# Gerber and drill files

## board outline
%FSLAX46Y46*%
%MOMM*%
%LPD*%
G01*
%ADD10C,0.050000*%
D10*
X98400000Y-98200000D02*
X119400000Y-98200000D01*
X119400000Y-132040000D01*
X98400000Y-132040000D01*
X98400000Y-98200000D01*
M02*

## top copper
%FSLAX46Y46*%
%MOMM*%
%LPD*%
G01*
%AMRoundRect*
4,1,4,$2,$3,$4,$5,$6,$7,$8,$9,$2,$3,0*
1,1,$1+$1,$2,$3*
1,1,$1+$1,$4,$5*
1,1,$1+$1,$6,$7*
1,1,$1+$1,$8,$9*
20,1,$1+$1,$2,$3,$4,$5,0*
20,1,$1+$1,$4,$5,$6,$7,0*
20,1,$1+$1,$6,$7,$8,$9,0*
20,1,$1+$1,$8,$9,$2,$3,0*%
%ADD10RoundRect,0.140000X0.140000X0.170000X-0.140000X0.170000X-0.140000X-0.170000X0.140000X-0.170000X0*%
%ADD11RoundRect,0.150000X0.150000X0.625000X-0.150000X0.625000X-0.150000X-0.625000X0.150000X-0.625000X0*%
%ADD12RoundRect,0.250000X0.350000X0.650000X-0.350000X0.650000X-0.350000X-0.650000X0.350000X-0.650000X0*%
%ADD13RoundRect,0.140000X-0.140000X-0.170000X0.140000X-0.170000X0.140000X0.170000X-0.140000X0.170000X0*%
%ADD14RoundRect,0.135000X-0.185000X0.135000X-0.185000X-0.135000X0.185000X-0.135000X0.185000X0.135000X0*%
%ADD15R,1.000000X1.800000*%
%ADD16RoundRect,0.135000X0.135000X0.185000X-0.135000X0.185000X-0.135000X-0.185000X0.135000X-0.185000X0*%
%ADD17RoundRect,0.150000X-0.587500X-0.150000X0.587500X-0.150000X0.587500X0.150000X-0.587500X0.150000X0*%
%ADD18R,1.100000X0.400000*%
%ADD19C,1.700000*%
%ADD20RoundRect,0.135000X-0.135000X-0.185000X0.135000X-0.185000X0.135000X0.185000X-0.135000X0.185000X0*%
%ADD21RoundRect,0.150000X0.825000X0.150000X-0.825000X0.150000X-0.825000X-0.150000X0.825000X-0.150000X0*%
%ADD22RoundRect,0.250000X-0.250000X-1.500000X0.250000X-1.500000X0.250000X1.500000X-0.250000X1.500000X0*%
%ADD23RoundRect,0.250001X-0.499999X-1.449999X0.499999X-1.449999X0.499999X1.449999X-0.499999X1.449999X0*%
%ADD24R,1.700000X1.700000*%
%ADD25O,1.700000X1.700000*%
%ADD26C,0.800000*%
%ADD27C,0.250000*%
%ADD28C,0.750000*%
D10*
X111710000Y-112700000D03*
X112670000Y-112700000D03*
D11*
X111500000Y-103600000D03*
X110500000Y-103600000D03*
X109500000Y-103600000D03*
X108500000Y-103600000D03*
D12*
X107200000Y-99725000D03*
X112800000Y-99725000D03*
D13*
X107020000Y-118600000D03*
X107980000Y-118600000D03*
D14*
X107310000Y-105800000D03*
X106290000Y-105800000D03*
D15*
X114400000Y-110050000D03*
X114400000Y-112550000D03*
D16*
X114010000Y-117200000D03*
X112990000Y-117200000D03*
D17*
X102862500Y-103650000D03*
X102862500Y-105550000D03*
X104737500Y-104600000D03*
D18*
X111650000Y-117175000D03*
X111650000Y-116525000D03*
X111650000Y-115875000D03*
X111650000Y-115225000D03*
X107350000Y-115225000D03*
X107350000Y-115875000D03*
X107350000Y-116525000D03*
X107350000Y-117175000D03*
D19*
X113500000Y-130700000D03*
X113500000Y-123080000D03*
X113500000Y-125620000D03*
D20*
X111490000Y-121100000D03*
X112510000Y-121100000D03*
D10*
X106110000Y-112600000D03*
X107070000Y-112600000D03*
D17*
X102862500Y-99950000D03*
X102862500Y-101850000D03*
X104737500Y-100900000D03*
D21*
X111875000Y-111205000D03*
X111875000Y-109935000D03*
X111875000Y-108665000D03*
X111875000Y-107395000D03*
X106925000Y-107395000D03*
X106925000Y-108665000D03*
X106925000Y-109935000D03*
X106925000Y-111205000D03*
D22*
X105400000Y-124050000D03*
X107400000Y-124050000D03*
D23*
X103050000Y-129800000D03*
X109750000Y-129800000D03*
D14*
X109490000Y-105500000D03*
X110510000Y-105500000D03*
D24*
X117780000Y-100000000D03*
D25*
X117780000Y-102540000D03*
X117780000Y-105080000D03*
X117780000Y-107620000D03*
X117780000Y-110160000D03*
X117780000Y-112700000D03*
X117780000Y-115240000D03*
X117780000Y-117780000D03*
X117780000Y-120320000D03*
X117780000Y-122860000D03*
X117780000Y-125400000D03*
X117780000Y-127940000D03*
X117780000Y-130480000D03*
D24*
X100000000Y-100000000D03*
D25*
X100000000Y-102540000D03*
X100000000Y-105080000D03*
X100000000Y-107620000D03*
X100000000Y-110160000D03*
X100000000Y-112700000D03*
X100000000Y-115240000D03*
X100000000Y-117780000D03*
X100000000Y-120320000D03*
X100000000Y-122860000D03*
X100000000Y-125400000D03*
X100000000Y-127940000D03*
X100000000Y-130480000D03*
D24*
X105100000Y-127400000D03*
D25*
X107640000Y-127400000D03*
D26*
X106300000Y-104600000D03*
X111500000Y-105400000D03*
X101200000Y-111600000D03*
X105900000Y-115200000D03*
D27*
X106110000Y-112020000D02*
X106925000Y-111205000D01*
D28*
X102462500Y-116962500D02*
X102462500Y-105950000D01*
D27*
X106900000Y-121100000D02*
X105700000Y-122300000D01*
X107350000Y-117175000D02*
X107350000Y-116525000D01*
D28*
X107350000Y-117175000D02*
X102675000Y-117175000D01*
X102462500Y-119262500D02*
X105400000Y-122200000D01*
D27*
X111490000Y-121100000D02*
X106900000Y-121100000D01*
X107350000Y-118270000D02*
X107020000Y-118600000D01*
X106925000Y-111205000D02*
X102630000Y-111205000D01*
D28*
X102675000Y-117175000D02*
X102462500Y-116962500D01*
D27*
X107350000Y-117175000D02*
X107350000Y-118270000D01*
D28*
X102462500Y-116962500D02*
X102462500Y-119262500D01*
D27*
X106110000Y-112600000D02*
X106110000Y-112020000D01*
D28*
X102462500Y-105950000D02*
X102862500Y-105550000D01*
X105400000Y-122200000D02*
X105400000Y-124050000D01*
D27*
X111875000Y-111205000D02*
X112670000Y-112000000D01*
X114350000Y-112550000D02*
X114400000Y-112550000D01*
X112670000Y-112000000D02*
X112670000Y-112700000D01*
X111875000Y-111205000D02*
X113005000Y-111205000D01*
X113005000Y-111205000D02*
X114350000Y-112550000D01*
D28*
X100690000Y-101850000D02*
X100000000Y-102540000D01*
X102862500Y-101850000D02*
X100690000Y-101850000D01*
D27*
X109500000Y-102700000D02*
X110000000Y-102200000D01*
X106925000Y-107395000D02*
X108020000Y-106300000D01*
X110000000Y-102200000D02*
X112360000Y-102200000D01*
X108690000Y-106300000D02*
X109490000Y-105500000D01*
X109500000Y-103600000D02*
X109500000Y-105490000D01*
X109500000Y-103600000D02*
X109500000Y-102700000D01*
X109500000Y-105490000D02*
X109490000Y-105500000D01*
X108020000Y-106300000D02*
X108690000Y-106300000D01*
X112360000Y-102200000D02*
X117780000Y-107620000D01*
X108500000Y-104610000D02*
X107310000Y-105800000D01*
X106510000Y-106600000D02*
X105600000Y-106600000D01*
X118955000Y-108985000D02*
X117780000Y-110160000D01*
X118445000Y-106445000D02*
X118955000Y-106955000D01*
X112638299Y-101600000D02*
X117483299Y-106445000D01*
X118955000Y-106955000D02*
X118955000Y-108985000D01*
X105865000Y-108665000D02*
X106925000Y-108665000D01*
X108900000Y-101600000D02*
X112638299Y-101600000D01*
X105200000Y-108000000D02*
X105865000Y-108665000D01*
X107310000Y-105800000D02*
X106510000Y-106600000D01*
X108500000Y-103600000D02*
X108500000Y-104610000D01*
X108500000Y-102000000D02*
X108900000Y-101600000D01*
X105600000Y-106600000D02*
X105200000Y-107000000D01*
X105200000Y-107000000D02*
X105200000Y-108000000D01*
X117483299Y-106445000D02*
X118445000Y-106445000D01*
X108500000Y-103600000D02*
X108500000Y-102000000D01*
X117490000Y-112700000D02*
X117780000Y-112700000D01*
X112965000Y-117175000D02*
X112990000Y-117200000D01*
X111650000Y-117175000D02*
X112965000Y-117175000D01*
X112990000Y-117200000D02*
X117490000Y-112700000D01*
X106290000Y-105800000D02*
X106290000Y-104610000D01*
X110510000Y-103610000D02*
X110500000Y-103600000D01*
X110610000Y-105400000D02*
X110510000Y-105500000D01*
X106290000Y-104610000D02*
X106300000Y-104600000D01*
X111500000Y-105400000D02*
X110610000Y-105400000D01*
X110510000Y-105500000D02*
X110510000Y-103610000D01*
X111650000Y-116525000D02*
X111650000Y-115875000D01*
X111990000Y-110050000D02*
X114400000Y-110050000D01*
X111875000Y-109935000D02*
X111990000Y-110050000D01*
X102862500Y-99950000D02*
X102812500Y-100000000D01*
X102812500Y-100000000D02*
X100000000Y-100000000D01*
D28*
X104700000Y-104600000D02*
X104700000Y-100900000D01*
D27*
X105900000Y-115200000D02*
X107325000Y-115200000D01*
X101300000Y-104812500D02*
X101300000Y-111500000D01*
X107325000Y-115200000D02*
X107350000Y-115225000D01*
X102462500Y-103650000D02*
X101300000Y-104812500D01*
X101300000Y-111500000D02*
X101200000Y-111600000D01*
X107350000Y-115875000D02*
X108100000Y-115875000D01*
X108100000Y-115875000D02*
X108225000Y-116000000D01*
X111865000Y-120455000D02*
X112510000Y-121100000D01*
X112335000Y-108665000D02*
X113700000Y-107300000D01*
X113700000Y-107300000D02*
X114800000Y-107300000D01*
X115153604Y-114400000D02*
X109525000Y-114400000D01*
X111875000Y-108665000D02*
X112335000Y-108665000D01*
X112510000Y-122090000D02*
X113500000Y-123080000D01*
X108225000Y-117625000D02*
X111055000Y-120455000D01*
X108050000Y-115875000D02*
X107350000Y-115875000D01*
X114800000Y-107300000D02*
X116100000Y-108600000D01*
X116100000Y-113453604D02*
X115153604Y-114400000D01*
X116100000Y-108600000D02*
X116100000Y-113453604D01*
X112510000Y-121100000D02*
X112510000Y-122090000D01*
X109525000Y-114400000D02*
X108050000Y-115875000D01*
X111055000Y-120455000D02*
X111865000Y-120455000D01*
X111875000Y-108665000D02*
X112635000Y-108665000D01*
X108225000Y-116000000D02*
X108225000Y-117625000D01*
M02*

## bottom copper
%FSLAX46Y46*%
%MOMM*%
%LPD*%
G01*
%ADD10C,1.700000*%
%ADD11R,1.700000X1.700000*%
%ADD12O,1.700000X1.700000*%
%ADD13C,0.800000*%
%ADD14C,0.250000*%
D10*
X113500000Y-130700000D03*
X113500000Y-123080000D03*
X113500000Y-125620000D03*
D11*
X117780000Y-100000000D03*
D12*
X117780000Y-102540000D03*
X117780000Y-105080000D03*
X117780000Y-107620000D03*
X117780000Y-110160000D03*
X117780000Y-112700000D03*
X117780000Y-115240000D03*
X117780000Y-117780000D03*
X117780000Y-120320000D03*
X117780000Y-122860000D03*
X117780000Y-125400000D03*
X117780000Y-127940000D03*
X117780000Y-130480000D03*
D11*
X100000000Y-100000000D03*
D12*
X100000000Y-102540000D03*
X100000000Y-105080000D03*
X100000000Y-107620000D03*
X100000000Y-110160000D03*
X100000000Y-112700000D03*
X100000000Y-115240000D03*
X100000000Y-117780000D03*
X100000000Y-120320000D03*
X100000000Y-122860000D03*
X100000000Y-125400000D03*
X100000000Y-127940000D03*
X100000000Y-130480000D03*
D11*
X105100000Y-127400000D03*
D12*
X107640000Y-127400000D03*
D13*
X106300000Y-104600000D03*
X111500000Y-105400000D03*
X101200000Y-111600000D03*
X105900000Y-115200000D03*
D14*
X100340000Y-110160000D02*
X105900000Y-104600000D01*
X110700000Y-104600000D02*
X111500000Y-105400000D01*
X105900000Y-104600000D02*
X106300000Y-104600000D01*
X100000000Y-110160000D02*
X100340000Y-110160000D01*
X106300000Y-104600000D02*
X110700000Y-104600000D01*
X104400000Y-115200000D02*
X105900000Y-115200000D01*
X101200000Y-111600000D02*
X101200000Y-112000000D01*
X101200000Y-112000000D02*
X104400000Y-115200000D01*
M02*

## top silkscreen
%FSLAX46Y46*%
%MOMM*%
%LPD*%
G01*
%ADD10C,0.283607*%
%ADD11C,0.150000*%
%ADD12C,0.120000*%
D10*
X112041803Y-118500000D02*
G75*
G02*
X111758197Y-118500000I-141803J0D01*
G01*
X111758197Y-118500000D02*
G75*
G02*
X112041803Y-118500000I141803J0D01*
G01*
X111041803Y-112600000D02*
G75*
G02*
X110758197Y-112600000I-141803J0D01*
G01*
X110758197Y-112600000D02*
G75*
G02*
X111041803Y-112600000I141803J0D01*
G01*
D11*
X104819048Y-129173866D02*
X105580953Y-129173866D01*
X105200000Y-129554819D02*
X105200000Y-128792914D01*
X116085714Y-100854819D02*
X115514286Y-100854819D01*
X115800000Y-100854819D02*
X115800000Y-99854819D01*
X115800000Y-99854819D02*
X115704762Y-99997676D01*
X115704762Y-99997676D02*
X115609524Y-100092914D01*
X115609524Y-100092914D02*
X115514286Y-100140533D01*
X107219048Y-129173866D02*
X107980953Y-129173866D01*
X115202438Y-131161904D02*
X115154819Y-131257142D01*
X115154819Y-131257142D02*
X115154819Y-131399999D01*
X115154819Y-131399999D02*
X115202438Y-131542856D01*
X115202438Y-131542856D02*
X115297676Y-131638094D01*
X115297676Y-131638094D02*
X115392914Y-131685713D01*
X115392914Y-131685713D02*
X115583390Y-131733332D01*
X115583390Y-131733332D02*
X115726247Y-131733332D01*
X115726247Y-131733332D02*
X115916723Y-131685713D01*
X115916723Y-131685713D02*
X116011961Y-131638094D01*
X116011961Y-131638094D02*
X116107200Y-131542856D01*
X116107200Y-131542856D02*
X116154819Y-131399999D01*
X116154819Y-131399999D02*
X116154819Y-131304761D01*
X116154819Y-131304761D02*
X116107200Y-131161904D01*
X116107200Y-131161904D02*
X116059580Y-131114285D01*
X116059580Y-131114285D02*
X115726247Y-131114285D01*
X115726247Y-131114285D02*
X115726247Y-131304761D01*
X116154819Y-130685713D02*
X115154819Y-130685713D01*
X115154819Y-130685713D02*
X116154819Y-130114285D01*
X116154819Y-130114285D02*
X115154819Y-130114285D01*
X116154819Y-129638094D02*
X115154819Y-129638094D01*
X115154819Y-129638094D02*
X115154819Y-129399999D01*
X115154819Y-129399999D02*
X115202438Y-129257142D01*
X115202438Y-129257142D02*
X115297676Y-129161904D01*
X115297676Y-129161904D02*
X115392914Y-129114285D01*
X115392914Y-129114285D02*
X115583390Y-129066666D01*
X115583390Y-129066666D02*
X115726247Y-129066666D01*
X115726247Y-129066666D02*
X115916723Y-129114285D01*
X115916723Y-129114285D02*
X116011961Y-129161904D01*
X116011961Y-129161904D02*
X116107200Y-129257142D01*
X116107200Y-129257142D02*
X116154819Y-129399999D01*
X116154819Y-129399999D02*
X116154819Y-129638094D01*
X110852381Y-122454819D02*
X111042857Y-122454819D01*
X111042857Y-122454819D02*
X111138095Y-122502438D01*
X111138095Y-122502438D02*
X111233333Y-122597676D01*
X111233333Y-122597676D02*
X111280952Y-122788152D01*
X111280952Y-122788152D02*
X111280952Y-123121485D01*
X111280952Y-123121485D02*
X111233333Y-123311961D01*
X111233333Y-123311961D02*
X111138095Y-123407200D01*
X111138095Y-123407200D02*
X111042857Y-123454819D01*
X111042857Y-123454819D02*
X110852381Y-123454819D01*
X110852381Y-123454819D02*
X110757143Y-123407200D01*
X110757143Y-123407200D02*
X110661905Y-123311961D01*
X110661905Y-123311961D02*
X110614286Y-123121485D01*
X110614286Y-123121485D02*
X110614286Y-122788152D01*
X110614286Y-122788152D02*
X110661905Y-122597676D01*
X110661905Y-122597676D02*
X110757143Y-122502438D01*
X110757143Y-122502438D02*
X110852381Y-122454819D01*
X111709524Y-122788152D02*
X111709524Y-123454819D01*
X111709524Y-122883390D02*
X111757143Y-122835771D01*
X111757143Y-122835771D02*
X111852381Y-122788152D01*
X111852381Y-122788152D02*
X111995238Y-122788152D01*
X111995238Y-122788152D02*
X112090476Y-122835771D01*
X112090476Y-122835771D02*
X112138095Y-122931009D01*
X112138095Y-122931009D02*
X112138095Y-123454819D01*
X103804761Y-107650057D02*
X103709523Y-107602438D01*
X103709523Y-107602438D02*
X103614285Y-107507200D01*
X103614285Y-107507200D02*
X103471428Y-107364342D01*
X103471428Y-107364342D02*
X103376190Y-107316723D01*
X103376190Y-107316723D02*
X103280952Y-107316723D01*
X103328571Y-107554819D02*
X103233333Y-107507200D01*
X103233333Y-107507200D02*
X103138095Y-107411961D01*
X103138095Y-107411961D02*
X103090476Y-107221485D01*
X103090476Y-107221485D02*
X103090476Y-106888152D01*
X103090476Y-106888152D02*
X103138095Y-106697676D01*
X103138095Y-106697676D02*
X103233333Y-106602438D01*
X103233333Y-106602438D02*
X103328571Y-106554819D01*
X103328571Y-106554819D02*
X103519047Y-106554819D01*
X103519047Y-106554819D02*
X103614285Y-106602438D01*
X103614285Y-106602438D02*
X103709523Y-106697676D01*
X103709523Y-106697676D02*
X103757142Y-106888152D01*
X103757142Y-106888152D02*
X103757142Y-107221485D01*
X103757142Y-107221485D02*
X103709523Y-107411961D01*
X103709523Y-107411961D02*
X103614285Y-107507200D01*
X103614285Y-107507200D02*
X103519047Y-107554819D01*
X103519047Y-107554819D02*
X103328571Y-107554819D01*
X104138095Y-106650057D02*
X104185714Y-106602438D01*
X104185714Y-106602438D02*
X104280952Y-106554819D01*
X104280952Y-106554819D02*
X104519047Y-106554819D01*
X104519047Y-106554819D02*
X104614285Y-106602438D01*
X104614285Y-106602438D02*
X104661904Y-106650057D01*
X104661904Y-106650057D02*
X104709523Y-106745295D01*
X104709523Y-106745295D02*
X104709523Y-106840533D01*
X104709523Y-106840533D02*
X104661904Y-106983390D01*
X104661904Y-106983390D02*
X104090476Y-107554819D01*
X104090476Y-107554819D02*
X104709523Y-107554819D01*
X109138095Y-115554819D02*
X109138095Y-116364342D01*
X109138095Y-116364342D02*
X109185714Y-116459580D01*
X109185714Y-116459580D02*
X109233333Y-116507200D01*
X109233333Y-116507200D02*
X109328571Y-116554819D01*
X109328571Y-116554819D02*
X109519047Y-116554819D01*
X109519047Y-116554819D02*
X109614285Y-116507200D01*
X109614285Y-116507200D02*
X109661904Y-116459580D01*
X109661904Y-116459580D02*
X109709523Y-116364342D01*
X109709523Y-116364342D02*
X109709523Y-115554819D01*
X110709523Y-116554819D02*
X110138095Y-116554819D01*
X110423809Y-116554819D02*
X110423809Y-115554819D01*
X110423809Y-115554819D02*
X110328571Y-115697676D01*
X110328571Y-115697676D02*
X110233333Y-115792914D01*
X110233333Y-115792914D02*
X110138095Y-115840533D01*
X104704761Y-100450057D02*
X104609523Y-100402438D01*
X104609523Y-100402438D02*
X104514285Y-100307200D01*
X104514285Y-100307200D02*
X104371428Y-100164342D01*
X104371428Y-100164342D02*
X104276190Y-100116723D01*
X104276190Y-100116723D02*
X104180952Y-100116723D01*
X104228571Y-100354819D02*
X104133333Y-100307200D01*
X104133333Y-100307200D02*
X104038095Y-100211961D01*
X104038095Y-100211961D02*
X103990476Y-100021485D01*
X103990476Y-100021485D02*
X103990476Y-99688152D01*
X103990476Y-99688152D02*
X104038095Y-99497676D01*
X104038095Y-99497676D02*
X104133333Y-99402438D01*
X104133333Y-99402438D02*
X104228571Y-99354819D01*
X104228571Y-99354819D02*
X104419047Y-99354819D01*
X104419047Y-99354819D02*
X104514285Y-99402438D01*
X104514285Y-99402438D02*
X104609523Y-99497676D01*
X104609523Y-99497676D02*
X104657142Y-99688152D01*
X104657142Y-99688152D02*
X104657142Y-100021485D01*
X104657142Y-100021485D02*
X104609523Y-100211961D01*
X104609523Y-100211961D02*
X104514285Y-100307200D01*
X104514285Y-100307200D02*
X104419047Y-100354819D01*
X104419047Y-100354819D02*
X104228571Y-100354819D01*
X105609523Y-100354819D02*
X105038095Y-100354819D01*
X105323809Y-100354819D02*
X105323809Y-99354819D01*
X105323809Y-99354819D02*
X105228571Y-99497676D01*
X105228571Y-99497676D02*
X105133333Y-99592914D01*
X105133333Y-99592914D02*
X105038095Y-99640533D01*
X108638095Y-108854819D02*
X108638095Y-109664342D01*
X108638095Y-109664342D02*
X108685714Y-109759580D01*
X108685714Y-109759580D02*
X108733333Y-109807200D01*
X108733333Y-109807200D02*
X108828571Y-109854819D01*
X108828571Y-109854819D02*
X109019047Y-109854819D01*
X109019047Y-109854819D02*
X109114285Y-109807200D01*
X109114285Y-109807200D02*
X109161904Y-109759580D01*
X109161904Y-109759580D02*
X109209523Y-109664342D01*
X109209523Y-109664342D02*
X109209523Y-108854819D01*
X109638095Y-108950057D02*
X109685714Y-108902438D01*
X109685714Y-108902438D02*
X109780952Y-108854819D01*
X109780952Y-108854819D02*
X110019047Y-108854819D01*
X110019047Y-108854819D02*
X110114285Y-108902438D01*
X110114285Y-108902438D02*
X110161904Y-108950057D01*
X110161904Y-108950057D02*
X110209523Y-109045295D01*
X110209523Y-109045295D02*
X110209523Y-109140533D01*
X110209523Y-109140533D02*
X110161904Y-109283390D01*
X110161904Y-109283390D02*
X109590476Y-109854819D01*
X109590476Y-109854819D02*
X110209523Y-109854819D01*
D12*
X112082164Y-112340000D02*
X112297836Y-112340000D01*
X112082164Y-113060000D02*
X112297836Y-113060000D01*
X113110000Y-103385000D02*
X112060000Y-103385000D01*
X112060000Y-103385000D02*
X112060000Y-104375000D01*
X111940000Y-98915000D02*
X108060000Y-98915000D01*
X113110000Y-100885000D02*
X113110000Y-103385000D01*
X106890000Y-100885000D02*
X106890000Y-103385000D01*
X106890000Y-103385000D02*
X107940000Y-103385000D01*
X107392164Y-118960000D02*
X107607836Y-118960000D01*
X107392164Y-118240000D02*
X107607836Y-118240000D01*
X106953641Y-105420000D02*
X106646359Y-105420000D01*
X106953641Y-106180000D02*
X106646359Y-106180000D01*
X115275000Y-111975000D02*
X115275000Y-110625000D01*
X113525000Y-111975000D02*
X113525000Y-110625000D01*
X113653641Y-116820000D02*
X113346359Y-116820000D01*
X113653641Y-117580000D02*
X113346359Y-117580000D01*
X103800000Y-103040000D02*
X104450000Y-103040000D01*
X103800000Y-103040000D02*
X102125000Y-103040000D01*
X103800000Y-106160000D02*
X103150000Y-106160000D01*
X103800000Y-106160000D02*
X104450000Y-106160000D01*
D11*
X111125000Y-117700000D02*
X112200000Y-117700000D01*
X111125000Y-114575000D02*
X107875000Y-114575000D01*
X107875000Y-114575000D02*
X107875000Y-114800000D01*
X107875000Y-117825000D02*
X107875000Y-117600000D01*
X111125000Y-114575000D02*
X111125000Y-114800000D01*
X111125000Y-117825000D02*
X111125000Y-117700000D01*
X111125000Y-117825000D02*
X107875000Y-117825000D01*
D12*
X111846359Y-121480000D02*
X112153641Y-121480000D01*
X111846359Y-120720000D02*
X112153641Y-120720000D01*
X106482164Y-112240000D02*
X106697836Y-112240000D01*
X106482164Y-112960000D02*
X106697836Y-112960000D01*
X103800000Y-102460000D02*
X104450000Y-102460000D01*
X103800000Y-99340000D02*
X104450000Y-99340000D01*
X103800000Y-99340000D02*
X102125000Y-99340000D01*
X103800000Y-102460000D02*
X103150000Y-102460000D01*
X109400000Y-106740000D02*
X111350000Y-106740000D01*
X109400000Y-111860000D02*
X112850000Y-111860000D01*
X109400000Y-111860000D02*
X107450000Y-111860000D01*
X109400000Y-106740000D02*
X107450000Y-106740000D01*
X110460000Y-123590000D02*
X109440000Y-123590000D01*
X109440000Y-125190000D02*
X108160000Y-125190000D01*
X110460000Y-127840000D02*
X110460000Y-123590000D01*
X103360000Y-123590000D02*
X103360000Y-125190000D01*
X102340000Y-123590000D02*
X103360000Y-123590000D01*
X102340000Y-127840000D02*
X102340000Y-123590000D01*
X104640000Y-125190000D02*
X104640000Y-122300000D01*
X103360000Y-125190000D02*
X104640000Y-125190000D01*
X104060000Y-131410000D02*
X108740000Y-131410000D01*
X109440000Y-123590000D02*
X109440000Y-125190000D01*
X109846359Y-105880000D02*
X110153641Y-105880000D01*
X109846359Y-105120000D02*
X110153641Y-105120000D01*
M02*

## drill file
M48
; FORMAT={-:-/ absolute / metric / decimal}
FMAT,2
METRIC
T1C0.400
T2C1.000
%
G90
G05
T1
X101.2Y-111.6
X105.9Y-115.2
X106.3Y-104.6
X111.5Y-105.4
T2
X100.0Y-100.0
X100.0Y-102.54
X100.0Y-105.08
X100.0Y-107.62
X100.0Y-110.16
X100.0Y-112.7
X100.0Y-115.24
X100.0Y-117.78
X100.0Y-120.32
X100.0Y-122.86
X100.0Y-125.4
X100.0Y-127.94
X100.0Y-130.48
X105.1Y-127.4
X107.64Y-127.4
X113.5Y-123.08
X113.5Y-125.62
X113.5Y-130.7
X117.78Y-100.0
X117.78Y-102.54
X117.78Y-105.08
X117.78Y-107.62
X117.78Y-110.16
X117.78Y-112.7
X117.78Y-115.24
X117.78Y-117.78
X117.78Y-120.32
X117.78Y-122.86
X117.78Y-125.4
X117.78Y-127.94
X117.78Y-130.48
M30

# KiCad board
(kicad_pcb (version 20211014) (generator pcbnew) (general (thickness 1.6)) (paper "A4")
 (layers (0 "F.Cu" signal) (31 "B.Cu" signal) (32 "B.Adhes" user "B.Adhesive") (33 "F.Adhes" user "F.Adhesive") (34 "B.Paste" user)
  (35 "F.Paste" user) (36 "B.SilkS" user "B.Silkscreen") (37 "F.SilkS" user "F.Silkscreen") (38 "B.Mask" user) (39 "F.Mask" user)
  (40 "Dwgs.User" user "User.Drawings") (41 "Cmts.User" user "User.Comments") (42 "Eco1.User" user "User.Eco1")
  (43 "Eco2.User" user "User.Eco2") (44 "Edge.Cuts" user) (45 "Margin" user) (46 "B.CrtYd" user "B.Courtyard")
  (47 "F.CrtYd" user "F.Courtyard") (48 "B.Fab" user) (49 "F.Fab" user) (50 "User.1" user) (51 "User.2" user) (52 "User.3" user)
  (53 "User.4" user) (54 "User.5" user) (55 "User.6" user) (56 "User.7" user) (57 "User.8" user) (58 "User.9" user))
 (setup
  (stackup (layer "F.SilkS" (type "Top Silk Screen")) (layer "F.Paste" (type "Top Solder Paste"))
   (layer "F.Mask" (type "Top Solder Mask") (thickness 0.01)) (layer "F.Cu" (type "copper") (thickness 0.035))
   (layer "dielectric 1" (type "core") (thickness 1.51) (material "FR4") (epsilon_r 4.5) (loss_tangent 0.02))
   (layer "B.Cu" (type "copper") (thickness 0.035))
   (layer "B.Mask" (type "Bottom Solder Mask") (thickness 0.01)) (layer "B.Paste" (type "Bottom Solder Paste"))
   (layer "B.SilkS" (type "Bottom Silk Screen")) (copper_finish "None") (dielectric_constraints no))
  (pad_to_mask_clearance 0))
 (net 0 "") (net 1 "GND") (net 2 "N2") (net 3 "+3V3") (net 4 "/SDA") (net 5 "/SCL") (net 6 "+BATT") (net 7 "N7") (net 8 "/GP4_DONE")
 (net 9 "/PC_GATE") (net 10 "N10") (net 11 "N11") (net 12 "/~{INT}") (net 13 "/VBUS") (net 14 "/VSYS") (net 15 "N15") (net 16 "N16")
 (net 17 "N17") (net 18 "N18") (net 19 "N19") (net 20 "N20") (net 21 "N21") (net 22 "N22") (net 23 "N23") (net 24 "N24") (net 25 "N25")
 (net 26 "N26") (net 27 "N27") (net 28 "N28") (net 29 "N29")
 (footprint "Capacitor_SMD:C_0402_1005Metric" (layer "F.Cu") (at 112.19 112.7)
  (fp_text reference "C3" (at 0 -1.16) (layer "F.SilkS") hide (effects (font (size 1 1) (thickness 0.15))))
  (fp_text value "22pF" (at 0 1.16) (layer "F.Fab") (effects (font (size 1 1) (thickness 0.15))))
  (fp_line (start -0.107836 -0.36) (end 0.107836 -0.36) (layer "F.SilkS") (width 0.12))
  (fp_line (start -0.107836 0.36) (end 0.107836 0.36) (layer "F.SilkS") (width 0.12))
  (pad "1" smd roundrect (at -0.48 0 180) (size 0.56 0.62) (layers "F.Cu" "F.Paste" "F.Mask") (roundrect_rratio 0.25) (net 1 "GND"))
  (pad "2" smd roundrect (at 0.48 0 180) (size 0.56 0.62) (layers "F.Cu" "F.Paste" "F.Mask") (roundrect_rratio 0.25) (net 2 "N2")))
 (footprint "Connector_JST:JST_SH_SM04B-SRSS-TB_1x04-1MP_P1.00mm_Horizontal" (layer "F.Cu") (at 110 101.6 180)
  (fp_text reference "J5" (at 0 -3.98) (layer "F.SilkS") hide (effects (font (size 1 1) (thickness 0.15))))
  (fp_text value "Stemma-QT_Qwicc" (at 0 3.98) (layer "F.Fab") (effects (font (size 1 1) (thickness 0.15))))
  (fp_line (start -3.11 -1.785) (end -2.06 -1.785) (layer "F.SilkS") (width 0.12))
  (fp_line (start -2.06 -1.785) (end -2.06 -2.775) (layer "F.SilkS") (width 0.12))
  (fp_line (start -1.94 2.685) (end 1.94 2.685) (layer "F.SilkS") (width 0.12))
  (fp_line (start -3.11 0.715) (end -3.11 -1.785) (layer "F.SilkS") (width 0.12))
  (fp_line (start 3.11 0.715) (end 3.11 -1.785) (layer "F.SilkS") (width 0.12))
  (fp_line (start 3.11 -1.785) (end 2.06 -1.785) (layer "F.SilkS") (width 0.12))
  (pad "1" smd roundrect (at -1.5 -2 180) (size 0.6 1.55) (layers "F.Cu" "F.Paste" "F.Mask") (roundrect_rratio 0.25) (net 1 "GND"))
  (pad "2" smd roundrect (at -0.5 -2 180) (size 0.6 1.55) (layers "F.Cu" "F.Paste" "F.Mask") (roundrect_rratio 0.25) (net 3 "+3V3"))
  (pad "3" smd roundrect (at 0.5 -2 180) (size 0.6 1.55) (layers "F.Cu" "F.Paste" "F.Mask") (roundrect_rratio 0.25) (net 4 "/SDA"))
  (pad "4" smd roundrect (at 1.5 -2 180) (size 0.6 1.55) (layers "F.Cu" "F.Paste" "F.Mask") (roundrect_rratio 0.25) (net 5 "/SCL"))
  (pad "MP" smd roundrect (at 2.8 1.875 180) (size 1.2 1.8) (layers "F.Cu" "F.Paste" "F.Mask") (roundrect_rratio 0.208333))
  (pad "MP" smd roundrect (at -2.8 1.875 180) (size 1.2 1.8) (layers "F.Cu" "F.Paste" "F.Mask") (roundrect_rratio 0.208333)))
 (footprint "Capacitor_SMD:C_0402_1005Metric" (layer "F.Cu") (at 107.5 118.6)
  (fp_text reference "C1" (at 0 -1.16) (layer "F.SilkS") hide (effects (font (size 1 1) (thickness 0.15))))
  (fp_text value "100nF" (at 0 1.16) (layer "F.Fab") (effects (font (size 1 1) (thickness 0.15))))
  (fp_line (start -0.107836 0.36) (end 0.107836 0.36) (layer "F.SilkS") (width 0.12))
  (fp_line (start -0.107836 -0.36) (end 0.107836 -0.36) (layer "F.SilkS") (width 0.12))
  (pad "1" smd roundrect (at -0.48 0) (size 0.56 0.62) (layers "F.Cu" "F.Paste" "F.Mask") (roundrect_rratio 0.25) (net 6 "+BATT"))
  (pad "2" smd roundrect (at 0.48 0) (size 0.56 0.62) (layers "F.Cu" "F.Paste" "F.Mask") (roundrect_rratio 0.25) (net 1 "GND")))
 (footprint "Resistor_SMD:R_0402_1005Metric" (layer "F.Cu") (at 106.8 105.8 180)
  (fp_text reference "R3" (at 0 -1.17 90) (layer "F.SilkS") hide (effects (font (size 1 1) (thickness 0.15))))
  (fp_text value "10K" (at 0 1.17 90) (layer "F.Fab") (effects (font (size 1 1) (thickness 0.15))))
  (fp_line (start -0.153641 0.38) (end 0.153641 0.38) (layer "F.SilkS") (width 0.12))
  (fp_line (start -0.153641 -0.38) (end 0.153641 -0.38) (layer "F.SilkS") (width 0.12))
  (pad "1" smd roundrect (at -0.51 0 270) (size 0.54 0.64) (layers "F.Cu" "F.Paste" "F.Mask") (roundrect_rratio 0.25) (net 5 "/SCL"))
  (pad "2" smd roundrect (at 0.51 0 270) (size 0.54 0.64) (layers "F.Cu" "F.Paste" "F.Mask") (roundrect_rratio 0.25) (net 3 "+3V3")))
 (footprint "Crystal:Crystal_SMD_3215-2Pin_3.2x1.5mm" (layer "F.Cu") (at 114.4 111.3 90)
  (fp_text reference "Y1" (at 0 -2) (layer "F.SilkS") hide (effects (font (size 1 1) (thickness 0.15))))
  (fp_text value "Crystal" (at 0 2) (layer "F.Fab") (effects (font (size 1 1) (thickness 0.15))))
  (fp_line (start -0.675 0.875) (end 0.675 0.875) (layer "F.SilkS") (width 0.12))
  (fp_line (start -0.675 -0.875) (end 0.675 -0.875) (layer "F.SilkS") (width 0.12))
  (pad "1" smd rect (at 1.25 0 180) (size 1 1.8) (layers "F.Cu" "F.Paste" "F.Mask") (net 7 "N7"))
  (pad "2" smd rect (at -1.25 0 180) (size 1 1.8) (layers "F.Cu" "F.Paste" "F.Mask") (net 2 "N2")))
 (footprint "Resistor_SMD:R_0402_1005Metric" (layer "F.Cu") (at 113.5 117.2 180)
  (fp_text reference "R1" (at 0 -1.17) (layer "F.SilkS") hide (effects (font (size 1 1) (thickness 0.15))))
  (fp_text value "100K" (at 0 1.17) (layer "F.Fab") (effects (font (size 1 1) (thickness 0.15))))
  (fp_line (start -0.153641 0.38) (end 0.153641 0.38) (layer "F.SilkS") (width 0.12))
  (fp_line (start -0.153641 -0.38) (end 0.153641 -0.38) (layer "F.SilkS") (width 0.12))
  (pad "1" smd roundrect (at -0.51 0 180) (size 0.54 0.64) (layers "F.Cu" "F.Paste" "F.Mask") (roundrect_rratio 0.25) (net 1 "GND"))
  (pad "2" smd roundrect (at 0.51 0 180) (size 0.54 0.64) (layers "F.Cu" "F.Paste" "F.Mask") (roundrect_rratio 0.25) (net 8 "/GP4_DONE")))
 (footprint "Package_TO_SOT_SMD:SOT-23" (layer "F.Cu") (at 103.8 104.6)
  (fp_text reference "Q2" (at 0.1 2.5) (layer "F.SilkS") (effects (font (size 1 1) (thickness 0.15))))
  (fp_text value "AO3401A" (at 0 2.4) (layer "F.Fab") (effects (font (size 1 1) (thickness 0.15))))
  (fp_line (start 0 -1.56) (end 0.65 -1.56) (layer "F.SilkS") (width 0.12))
  (fp_line (start 0 -1.56) (end -1.675 -1.56) (layer "F.SilkS") (width 0.12))
  (fp_line (start 0 1.56) (end -0.65 1.56) (layer "F.SilkS") (width 0.12))
  (fp_line (start 0 1.56) (end 0.65 1.56) (layer "F.SilkS") (width 0.12))
  (pad "1" smd roundrect (at -0.9375 -0.95) (size 1.475 0.6) (layers "F.Cu" "F.Paste" "F.Mask") (roundrect_rratio 0.25) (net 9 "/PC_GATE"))
  (pad "2" smd roundrect (at -0.9375 0.95) (size 1.475 0.6) (layers "F.Cu" "F.Paste" "F.Mask") (roundrect_rratio 0.25) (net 6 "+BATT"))
  (pad "3" smd roundrect (at 0.9375 0) (size 1.475 0.6) (layers "F.Cu" "F.Paste" "F.Mask") (roundrect_rratio 0.25) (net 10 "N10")))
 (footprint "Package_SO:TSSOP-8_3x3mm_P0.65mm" (layer "F.Cu") (at 109.5 116.2 180)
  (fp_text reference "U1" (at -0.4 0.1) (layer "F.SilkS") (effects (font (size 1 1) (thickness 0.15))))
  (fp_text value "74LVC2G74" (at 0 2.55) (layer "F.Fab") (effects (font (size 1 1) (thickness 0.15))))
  (fp_line (start -1.625 -1.5) (end -2.7 -1.5) (layer "F.SilkS") (width 0.15))
  (fp_line (start -1.625 1.625) (end 1.625 1.625) (layer "F.SilkS") (width 0.15))
  (fp_line (start 1.625 1.625) (end 1.625 1.4) (layer "F.SilkS") (width 0.15))
  (fp_line (start 1.625 -1.625) (end 1.625 -1.4) (layer "F.SilkS") (width 0.15))
  (fp_line (start -1.625 1.625) (end -1.625 1.4) (layer "F.SilkS") (width 0.15))
  (fp_line (start -1.625 -1.625) (end -1.625 -1.5) (layer "F.SilkS") (width 0.15))
  (fp_line (start -1.625 -1.625) (end 1.625 -1.625) (layer "F.SilkS") (width 0.15))
  (pad "1" smd rect (at -2.15 -0.975 180) (size 1.1 0.4) (layers "F.Cu" "F.Paste" "F.Mask") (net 8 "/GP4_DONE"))
  (pad "2" smd rect (at -2.15 -0.325 180) (size 1.1 0.4) (layers "F.Cu" "F.Paste" "F.Mask") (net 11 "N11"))
  (pad "3" smd rect (at -2.15 0.325 180) (size 1.1 0.4) (layers "F.Cu" "F.Paste" "F.Mask") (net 11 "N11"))
  (pad "4" smd rect (at -2.15 0.975 180) (size 1.1 0.4) (layers "F.Cu" "F.Paste" "F.Mask") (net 1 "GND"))
  (pad "5" smd rect (at 2.15 0.975 180) (size 1.1 0.4) (layers "F.Cu" "F.Paste" "F.Mask") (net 9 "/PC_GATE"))
  (pad "6" smd rect (at 2.15 0.325 180) (size 1.1 0.4) (layers "F.Cu" "F.Paste" "F.Mask") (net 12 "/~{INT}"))
  (pad "7" smd rect (at 2.15 -0.325 180) (size 1.1 0.4) (layers "F.Cu" "F.Paste" "F.Mask") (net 6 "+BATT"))
  (pad "8" smd rect (at 2.15 -0.975 180) (size 1.1 0.4) (layers "F.Cu" "F.Paste" "F.Mask") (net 6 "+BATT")))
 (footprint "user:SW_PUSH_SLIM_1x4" (layer "F.Cu") (at 113.5 130.7 90)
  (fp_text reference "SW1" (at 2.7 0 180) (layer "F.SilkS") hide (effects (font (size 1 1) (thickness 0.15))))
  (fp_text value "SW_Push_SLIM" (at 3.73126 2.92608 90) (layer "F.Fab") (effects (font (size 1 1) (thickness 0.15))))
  (pad "1" thru_hole circle (at 0 0 90) (size 1.7 1.7) (drill 1) (layers *.Cu *.Mask) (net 1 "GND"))
  (pad "2" thru_hole circle (at 7.62 0 90) (size 1.7 1.7) (drill 1) (layers *.Cu *.Mask) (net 12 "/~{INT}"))
  (pad "3" thru_hole circle (at 5.08 0 90) (size 1.7 1.7) (drill 1) (layers *.Cu *.Mask) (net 1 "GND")))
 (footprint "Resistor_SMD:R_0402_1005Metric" (layer "F.Cu") (at 112 121.1)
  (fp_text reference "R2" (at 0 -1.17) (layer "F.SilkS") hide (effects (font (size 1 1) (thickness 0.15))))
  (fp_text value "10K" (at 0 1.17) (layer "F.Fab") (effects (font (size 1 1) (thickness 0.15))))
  (fp_line (start -0.153641 0.38) (end 0.153641 0.38) (layer "F.SilkS") (width 0.12))
  (fp_line (start -0.153641 -0.38) (end 0.153641 -0.38) (layer "F.SilkS") (width 0.12))
  (pad "1" smd roundrect (at -0.51 0) (size 0.54 0.64) (layers "F.Cu" "F.Paste" "F.Mask") (roundrect_rratio 0.25) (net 6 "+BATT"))
  (pad "2" smd roundrect (at 0.51 0) (size 0.54 0.64) (layers "F.Cu" "F.Paste" "F.Mask") (roundrect_rratio 0.25) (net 12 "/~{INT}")))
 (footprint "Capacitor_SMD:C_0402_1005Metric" (layer "F.Cu") (at 106.59 112.6)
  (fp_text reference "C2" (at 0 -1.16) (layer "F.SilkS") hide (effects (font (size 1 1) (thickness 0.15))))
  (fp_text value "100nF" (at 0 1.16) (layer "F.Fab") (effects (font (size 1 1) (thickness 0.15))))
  (fp_line (start -0.107836 -0.36) (end 0.107836 -0.36) (layer "F.SilkS") (width 0.12))
  (fp_line (start -0.107836 0.36) (end 0.107836 0.36) (layer "F.SilkS") (width 0.12))
  (pad "1" smd roundrect (at -0.48 0 180) (size 0.56 0.62) (layers "F.Cu" "F.Paste" "F.Mask") (roundrect_rratio 0.25) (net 6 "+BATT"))
  (pad "2" smd roundrect (at 0.48 0 180) (size 0.56 0.62) (layers "F.Cu" "F.Paste" "F.Mask") (roundrect_rratio 0.25) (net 1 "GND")))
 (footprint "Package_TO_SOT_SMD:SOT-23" (layer "F.Cu") (at 103.8 100.9)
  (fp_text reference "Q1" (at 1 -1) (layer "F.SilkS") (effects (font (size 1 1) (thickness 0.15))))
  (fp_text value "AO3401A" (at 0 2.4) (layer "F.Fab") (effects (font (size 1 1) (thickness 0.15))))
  (fp_line (start 0 1.56) (end 0.65 1.56) (layer "F.SilkS") (width 0.12))
  (fp_line (start 0 -1.56) (end 0.65 -1.56) (layer "F.SilkS") (width 0.12))
  (fp_line (start 0 -1.56) (end -1.675 -1.56) (layer "F.SilkS") (width 0.12))
  (fp_line (start 0 1.56) (end -0.65 1.56) (layer "F.SilkS") (width 0.12))
  (pad "1" smd roundrect (at -0.9375 -0.95) (size 1.475 0.6) (layers "F.Cu" "F.Paste" "F.Mask") (roundrect_rratio 0.25) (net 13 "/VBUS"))
  (pad "2" smd roundrect (at -0.9375 0.95) (size 1.475 0.6) (layers "F.Cu" "F.Paste" "F.Mask") (roundrect_rratio 0.25) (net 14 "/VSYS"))
  (pad "3" smd roundrect (at 0.9375 0) (size 1.475 0.6) (layers "F.Cu" "F.Paste" "F.Mask") (roundrect_rratio 0.25) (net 10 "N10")))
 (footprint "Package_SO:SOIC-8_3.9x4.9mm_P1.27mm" (layer "F.Cu") (at 109.4 109.3 180)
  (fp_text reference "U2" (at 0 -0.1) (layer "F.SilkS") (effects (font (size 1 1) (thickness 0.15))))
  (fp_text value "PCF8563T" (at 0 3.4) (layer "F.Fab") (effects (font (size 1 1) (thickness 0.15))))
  (fp_line (start 0 2.56) (end -1.95 2.56) (layer "F.SilkS") (width 0.12))
  (fp_line (start 0 -2.56) (end -3.45 -2.56) (layer "F.SilkS") (width 0.12))
  (fp_line (start 0 -2.56) (end 1.95 -2.56) (layer "F.SilkS") (width 0.12))
  (fp_line (start 0 2.56) (end 1.95 2.56) (layer "F.SilkS") (width 0.12))
  (pad "1" smd roundrect (at -2.475 -1.905 180) (size 1.95 0.6) (layers "F.Cu" "F.Paste" "F.Mask") (roundrect_rratio 0.25) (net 2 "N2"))
  (pad "2" smd roundrect (at -2.475 -0.635 180) (size 1.95 0.6) (layers "F.Cu" "F.Paste" "F.Mask") (roundrect_rratio 0.25) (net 7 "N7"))
  (pad "3" smd roundrect (at -2.475 0.635 180) (size 1.95 0.6) (layers "F.Cu" "F.Paste" "F.Mask") (roundrect_rratio 0.25) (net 12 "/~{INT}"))
  (pad "4" smd roundrect (at -2.475 1.905 180) (size 1.95 0.6) (layers "F.Cu" "F.Paste" "F.Mask") (roundrect_rratio 0.25) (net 1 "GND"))
  (pad "5" smd roundrect (at 2.475 1.905 180) (size 1.95 0.6) (layers "F.Cu" "F.Paste" "F.Mask") (roundrect_rratio 0.25) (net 4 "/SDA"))
  (pad "6" smd roundrect (at 2.475 0.635 180) (size 1.95 0.6) (layers "F.Cu" "F.Paste" "F.Mask") (roundrect_rratio 0.25) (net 5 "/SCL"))
  (pad "7" smd roundrect (at 2.475 -0.635 180) (size 1.95 0.6) (layers "F.Cu" "F.Paste" "F.Mask") (roundrect_rratio 0.25) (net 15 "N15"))
  (pad "8" smd roundrect (at 2.475 -1.905 180) (size 1.95 0.6) (layers "F.Cu" "F.Paste" "F.Mask") (roundrect_rratio 0.25) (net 6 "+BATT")))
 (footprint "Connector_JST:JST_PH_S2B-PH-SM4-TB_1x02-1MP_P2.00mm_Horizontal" (layer "F.Cu") (at 106.4 126.9)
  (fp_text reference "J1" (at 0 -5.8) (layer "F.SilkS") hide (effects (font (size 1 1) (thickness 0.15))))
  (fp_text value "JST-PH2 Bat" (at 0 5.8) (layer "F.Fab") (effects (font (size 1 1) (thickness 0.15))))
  (fp_line (start 4.06 -3.31) (end 3.04 -3.31) (layer "F.SilkS") (width 0.12))
  (fp_line (start 3.04 -1.71) (end 1.76 -1.71) (layer "F.SilkS") (width 0.12))
  (fp_line (start 4.06 0.94) (end 4.06 -3.31) (layer "F.SilkS") (width 0.12))
  (fp_line (start -3.04 -3.31) (end -3.04 -1.71) (layer "F.SilkS") (width 0.12))
  (fp_line (start -4.06 -3.31) (end -3.04 -3.31) (layer "F.SilkS") (width 0.12))
  (fp_line (start -4.06 0.94) (end -4.06 -3.31) (layer "F.SilkS") (width 0.12))
  (fp_line (start -1.76 -1.71) (end -1.76 -4.6) (layer "F.SilkS") (width 0.12))
  (fp_line (start -3.04 -1.71) (end -1.76 -1.71) (layer "F.SilkS") (width 0.12))
  (fp_line (start -2.34 4.51) (end 2.34 4.51) (layer "F.SilkS") (width 0.12))
  (fp_line (start 3.04 -3.31) (end 3.04 -1.71) (layer "F.SilkS") (width 0.12))
  (pad "1" smd roundrect (at -1 -2.85) (size 1 3.5) (layers "F.Cu" "F.Paste" "F.Mask") (roundrect_rratio 0.25) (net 6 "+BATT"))
  (pad "2" smd roundrect (at 1 -2.85) (size 1 3.5) (layers "F.Cu" "F.Paste" "F.Mask") (roundrect_rratio 0.25) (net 1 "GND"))
  (pad "MP" smd roundrect (at -3.35 2.9) (size 1.5 3.4) (layers "F.Cu" "F.Paste" "F.Mask") (roundrect_rratio 0.1666673333))
  (pad "MP" smd roundrect (at 3.35 2.9) (size 1.5 3.4) (layers "F.Cu" "F.Paste" "F.Mask") (roundrect_rratio 0.1666673333)))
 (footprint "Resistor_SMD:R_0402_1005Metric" (layer "F.Cu") (at 110 105.5)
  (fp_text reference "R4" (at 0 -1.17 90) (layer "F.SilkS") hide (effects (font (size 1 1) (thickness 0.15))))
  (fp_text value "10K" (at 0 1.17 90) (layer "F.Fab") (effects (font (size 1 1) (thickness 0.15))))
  (fp_line (start -0.153641 0.38) (end 0.153641 0.38) (layer "F.SilkS") (width 0.12))
  (fp_line (start -0.153641 -0.38) (end 0.153641 -0.38) (layer "F.SilkS") (width 0.12))
  (pad "1" smd roundrect (at -0.51 0 270) (size 0.54 0.64) (layers "F.Cu" "F.Paste" "F.Mask") (roundrect_rratio 0.25) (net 4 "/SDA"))
  (pad "2" smd roundrect (at 0.51 0 270) (size 0.54 0.64) (layers "F.Cu" "F.Paste" "F.Mask") (roundrect_rratio 0.25) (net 3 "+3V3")))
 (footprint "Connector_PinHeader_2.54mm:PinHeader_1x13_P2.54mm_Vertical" (layer "B.Cu") (at 117.78 100 180)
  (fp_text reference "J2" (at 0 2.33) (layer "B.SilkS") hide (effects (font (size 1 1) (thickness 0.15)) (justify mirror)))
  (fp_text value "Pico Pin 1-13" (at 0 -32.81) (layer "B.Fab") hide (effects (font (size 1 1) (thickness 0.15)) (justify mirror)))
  (pad "1" thru_hole rect (at 0 0 180) (size 1.7 1.7) (drill 1) (layers *.Cu *.Mask) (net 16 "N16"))
  (pad "2" thru_hole oval (at 0 -2.54 180) (size 1.7 1.7) (drill 1) (layers *.Cu *.Mask) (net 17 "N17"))
  (pad "3" thru_hole oval (at 0 -5.08 180) (size 1.7 1.7) (drill 1) (layers *.Cu *.Mask) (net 1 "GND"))
  (pad "4" thru_hole oval (at 0 -7.62 180) (size 1.7 1.7) (drill 1) (layers *.Cu *.Mask) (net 4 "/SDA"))
  (pad "5" thru_hole oval (at 0 -10.16 180) (size 1.7 1.7) (drill 1) (layers *.Cu *.Mask) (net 5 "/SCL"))
  (pad "6" thru_hole oval (at 0 -12.7 180) (size 1.7 1.7) (drill 1) (layers *.Cu *.Mask) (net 8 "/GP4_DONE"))
  (pad "7" thru_hole oval (at 0 -15.24 180) (size 1.7 1.7) (drill 1) (layers *.Cu *.Mask) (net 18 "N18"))
  (pad "8" thru_hole oval (at 0 -17.78 180) (size 1.7 1.7) (drill 1) (layers *.Cu *.Mask) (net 1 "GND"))
  (pad "9" thru_hole oval (at 0 -20.32 180) (size 1.7 1.7) (drill 1) (layers *.Cu *.Mask) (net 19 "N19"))
  (pad "10" thru_hole oval (at 0 -22.86 180) (size 1.7 1.7) (drill 1) (layers *.Cu *.Mask) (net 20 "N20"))
  (pad "11" thru_hole oval (at 0 -25.4 180) (size 1.7 1.7) (drill 1) (layers *.Cu *.Mask) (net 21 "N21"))
  (pad "12" thru_hole oval (at 0 -27.94 180) (size 1.7 1.7) (drill 1) (layers *.Cu *.Mask) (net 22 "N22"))
  (pad "13" thru_hole oval (at 0 -30.48 180) (size 1.7 1.7) (drill 1) (layers *.Cu *.Mask) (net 1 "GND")))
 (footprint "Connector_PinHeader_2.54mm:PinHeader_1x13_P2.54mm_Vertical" (layer "B.Cu") (at 100 100 180)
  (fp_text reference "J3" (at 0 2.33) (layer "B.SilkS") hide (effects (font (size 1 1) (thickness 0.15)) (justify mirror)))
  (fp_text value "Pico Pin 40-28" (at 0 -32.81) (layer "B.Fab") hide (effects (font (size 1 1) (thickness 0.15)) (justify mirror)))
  (pad "1" thru_hole rect (at 0 0 180) (size 1.7 1.7) (drill 1) (layers *.Cu *.Mask) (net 13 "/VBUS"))
  (pad "2" thru_hole oval (at 0 -2.54 180) (size 1.7 1.7) (drill 1) (layers *.Cu *.Mask) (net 14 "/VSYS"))
  (pad "3" thru_hole oval (at 0 -5.08 180) (size 1.7 1.7) (drill 1) (layers *.Cu *.Mask) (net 1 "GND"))
  (pad "4" thru_hole oval (at 0 -7.62 180) (size 1.7 1.7) (drill 1) (layers *.Cu *.Mask) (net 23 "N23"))
  (pad "5" thru_hole oval (at 0 -10.16 180) (size 1.7 1.7) (drill 1) (layers *.Cu *.Mask) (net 3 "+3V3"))
  (pad "6" thru_hole oval (at 0 -12.7 180) (size 1.7 1.7) (drill 1) (layers *.Cu *.Mask) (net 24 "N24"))
  (pad "7" thru_hole oval (at 0 -15.24 180) (size 1.7 1.7) (drill 1) (layers *.Cu *.Mask) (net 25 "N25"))
  (pad "8" thru_hole oval (at 0 -17.78 180) (size 1.7 1.7) (drill 1) (layers *.Cu *.Mask) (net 1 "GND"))
  (pad "9" thru_hole oval (at 0 -20.32 180) (size 1.7 1.7) (drill 1) (layers *.Cu *.Mask) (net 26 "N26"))
  (pad "10" thru_hole oval (at 0 -22.86 180) (size 1.7 1.7) (drill 1) (layers *.Cu *.Mask) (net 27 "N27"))
  (pad "11" thru_hole oval (at 0 -25.4 180) (size 1.7 1.7) (drill 1) (layers *.Cu *.Mask) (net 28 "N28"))
  (pad "12" thru_hole oval (at 0 -27.94 180) (size 1.7 1.7) (drill 1) (layers *.Cu *.Mask) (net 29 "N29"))
  (pad "13" thru_hole oval (at 0 -30.48 180) (size 1.7 1.7) (drill 1) (layers *.Cu *.Mask) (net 1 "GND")))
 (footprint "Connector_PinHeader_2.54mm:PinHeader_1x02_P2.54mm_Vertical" (layer "B.Cu") (at 105.1 127.4 -90)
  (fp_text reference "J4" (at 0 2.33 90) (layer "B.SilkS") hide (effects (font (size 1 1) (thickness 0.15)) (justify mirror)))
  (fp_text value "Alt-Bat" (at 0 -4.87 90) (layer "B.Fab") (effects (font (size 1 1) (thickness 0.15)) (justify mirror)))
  (pad "1" thru_hole rect (at 0 0 270) (size 1.7 1.7) (drill 1) (layers *.Cu *.Mask) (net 1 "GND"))
  (pad "2" thru_hole oval (at 0 -2.54 270) (size 1.7 1.7) (drill 1) (layers *.Cu *.Mask) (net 1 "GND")))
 (gr_circle (center 111.9 118.5) (end 111.9 118.276393) (layer "F.SilkS") (width 0.12) (fill solid))
 (gr_circle (center 110.9 112.6) (end 110.9 112.823607) (layer "F.SilkS") (width 0.12) (fill solid))
 (gr_rect (start 98.4 98.2) (end 119.4 132.04) (layer "Edge.Cuts") (width 0.05) (fill none))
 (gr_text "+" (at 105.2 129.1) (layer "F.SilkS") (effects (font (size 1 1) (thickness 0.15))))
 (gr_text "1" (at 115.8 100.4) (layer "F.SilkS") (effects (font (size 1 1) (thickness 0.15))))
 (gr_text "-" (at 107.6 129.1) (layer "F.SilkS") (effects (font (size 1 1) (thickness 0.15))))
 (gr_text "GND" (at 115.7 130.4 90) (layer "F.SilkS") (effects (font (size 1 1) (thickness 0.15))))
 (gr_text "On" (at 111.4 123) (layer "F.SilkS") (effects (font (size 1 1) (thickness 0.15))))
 (segment (start 106.11 112.02) (end 106.925 111.205) (width 0.25) (layer "F.Cu") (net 6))
 (segment (start 102.4625 116.9625) (end 102.4625 105.95) (width 0.75) (layer "F.Cu") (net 6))
 (segment (start 106.9 121.1) (end 105.7 122.3) (width 0.25) (layer "F.Cu") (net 6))
 (segment (start 107.35 117.175) (end 107.35 116.525) (width 0.25) (layer "F.Cu") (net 6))
 (segment (start 107.35 117.175) (end 102.675 117.175) (width 0.75) (layer "F.Cu") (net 6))
 (segment (start 102.4625 119.2625) (end 105.4 122.2) (width 0.75) (layer "F.Cu") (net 6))
 (segment (start 111.49 121.1) (end 106.9 121.1) (width 0.25) (layer "F.Cu") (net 6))
 (segment (start 107.35 118.27) (end 107.02 118.6) (width 0.25) (layer "F.Cu") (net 6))
 (segment (start 106.925 111.205) (end 102.63 111.205) (width 0.25) (layer "F.Cu") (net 6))
 (segment (start 102.675 117.175) (end 102.4625 116.9625) (width 0.75) (layer "F.Cu") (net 6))
 (segment (start 107.35 117.175) (end 107.35 118.27) (width 0.25) (layer "F.Cu") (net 6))
 (segment (start 102.4625 116.9625) (end 102.4625 119.2625) (width 0.75) (layer "F.Cu") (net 6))
 (segment (start 106.11 112.6) (end 106.11 112.02) (width 0.25) (layer "F.Cu") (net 6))
 (segment (start 102.4625 105.95) (end 102.8625 105.55) (width 0.75) (layer "F.Cu") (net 6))
 (segment (start 105.4 122.2) (end 105.4 124.05) (width 0.75) (layer "F.Cu") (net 6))
 (segment (start 111.875 111.205) (end 112.67 112) (width 0.25) (layer "F.Cu") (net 2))
 (segment (start 114.35 112.55) (end 114.4 112.55) (width 0.25) (layer "F.Cu") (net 2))
 (segment (start 112.67 112) (end 112.67 112.7) (width 0.25) (layer "F.Cu") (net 2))
 (segment (start 111.875 111.205) (end 113.005 111.205) (width 0.25) (layer "F.Cu") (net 2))
 (segment (start 113.005 111.205) (end 114.35 112.55) (width 0.25) (layer "F.Cu") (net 2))
 (segment (start 100.69 101.85) (end 100 102.54) (width 0.75) (layer "F.Cu") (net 14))
 (segment (start 102.8625 101.85) (end 100.69 101.85) (width 0.75) (layer "F.Cu") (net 14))
 (segment (start 109.5 102.7) (end 110 102.2) (width 0.25) (layer "F.Cu") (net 4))
 (segment (start 106.925 107.395) (end 108.02 106.3) (width 0.25) (layer "F.Cu") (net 4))
 (segment (start 110 102.2) (end 112.36 102.2) (width 0.25) (layer "F.Cu") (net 4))
 (segment (start 108.69 106.3) (end 109.49 105.5) (width 0.25) (layer "F.Cu") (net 4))
 (segment (start 109.5 103.6) (end 109.5 105.49) (width 0.25) (layer "F.Cu") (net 4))
 (segment (start 109.5 103.6) (end 109.5 102.7) (width 0.25) (layer "F.Cu") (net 4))
 (segment (start 109.5 105.49) (end 109.49 105.5) (width 0.25) (layer "F.Cu") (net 4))
 (segment (start 108.02 106.3) (end 108.69 106.3) (width 0.25) (layer "F.Cu") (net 4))
 (segment (start 112.36 102.2) (end 117.78 107.62) (width 0.25) (layer "F.Cu") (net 4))
 (segment (start 108.5 104.61) (end 107.31 105.8) (width 0.25) (layer "F.Cu") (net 5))
 (segment (start 106.51 106.6) (end 105.6 106.6) (width 0.25) (layer "F.Cu") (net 5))
 (segment (start 118.955 108.985) (end 117.78 110.16) (width 0.25) (layer "F.Cu") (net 5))
 (segment (start 118.445 106.445) (end 118.955 106.955) (width 0.25) (layer "F.Cu") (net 5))
 (segment (start 112.638299 101.6) (end 117.483299 106.445) (width 0.25) (layer "F.Cu") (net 5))
 (segment (start 118.955 106.955) (end 118.955 108.985) (width 0.25) (layer "F.Cu") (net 5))
 (segment (start 105.865 108.665) (end 106.925 108.665) (width 0.25) (layer "F.Cu") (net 5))
 (segment (start 108.9 101.6) (end 112.638299 101.6) (width 0.25) (layer "F.Cu") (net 5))
 (segment (start 105.2 108) (end 105.865 108.665) (width 0.25) (layer "F.Cu") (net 5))
 (segment (start 107.31 105.8) (end 106.51 106.6) (width 0.25) (layer "F.Cu") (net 5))
 (segment (start 108.5 103.6) (end 108.5 104.61) (width 0.25) (layer "F.Cu") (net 5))
 (segment (start 108.5 102) (end 108.9 101.6) (width 0.25) (layer "F.Cu") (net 5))
 (segment (start 105.6 106.6) (end 105.2 107) (width 0.25) (layer "F.Cu") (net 5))
 (segment (start 105.2 107) (end 105.2 108) (width 0.25) (layer "F.Cu") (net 5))
 (segment (start 117.483299 106.445) (end 118.445 106.445) (width 0.25) (layer "F.Cu") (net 5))
 (segment (start 108.5 103.6) (end 108.5 102) (width 0.25) (layer "F.Cu") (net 5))
 (segment (start 117.49 112.7) (end 117.78 112.7) (width 0.25) (layer "F.Cu") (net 8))
 (segment (start 112.965 117.175) (end 112.99 117.2) (width 0.25) (layer "F.Cu") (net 8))
 (segment (start 111.65 117.175) (end 112.965 117.175) (width 0.25) (layer "F.Cu") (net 8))
 (segment (start 112.99 117.2) (end 117.49 112.7) (width 0.25) (layer "F.Cu") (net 8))
 (segment (start 106.29 105.8) (end 106.29 104.61) (width 0.25) (layer "F.Cu") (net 3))
 (segment (start 110.51 103.61) (end 110.5 103.6) (width 0.25) (layer "F.Cu") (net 3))
 (segment (start 110.61 105.4) (end 110.51 105.5) (width 0.25) (layer "F.Cu") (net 3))
 (segment (start 106.29 104.61) (end 106.3 104.6) (width 0.25) (layer "F.Cu") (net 3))
 (segment (start 111.5 105.4) (end 110.61 105.4) (width 0.25) (layer "F.Cu") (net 3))
 (segment (start 110.51 105.5) (end 110.51 103.61) (width 0.25) (layer "F.Cu") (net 3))
 (via (at 106.3 104.6) (size 0.8) (drill 0.4) (layers "F.Cu" "B.Cu") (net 3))
 (via (at 111.5 105.4) (size 0.8) (drill 0.4) (layers "F.Cu" "B.Cu") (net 3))
 (segment (start 100.34 110.16) (end 105.9 104.6) (width 0.25) (layer "B.Cu") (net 3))
 (segment (start 110.7 104.6) (end 111.5 105.4) (width 0.25) (layer "B.Cu") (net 3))
 (segment (start 105.9 104.6) (end 106.3 104.6) (width 0.25) (layer "B.Cu") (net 3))
 (segment (start 100 110.16) (end 100.34 110.16) (width 0.25) (layer "B.Cu") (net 3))
 (segment (start 106.3 104.6) (end 110.7 104.6) (width 0.25) (layer "B.Cu") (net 3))
 (segment (start 111.65 116.525) (end 111.65 115.875) (width 0.25) (layer "F.Cu") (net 11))
 (segment (start 111.99 110.05) (end 114.4 110.05) (width 0.25) (layer "F.Cu") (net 7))
 (segment (start 111.875 109.935) (end 111.99 110.05) (width 0.25) (layer "F.Cu") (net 7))
 (segment (start 102.8625 99.95) (end 102.8125 100) (width 0.25) (layer "F.Cu") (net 13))
 (segment (start 102.8125 100) (end 100 100) (width 0.25) (layer "F.Cu") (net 13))
 (segment (start 104.7 104.6) (end 104.7 100.9) (width 0.75) (layer "F.Cu") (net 10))
 (segment (start 105.9 115.2) (end 107.325 115.2) (width 0.25) (layer "F.Cu") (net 9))
 (segment (start 101.3 104.8125) (end 101.3 111.5) (width 0.25) (layer "F.Cu") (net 9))
 (segment (start 107.325 115.2) (end 107.35 115.225) (width 0.25) (layer "F.Cu") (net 9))
 (segment (start 102.4625 103.65) (end 101.3 104.8125) (width 0.25) (layer "F.Cu") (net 9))
 (segment (start 101.3 111.5) (end 101.2 111.6) (width 0.25) (layer "F.Cu") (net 9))
 (via (at 101.2 111.6) (size 0.8) (drill 0.4) (layers "F.Cu" "B.Cu") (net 9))
 (via (at 105.9 115.2) (size 0.8) (drill 0.4) (layers "F.Cu" "B.Cu") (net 9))
 (segment (start 104.4 115.2) (end 105.9 115.2) (width 0.25) (layer "B.Cu") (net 9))
 (segment (start 101.2 111.6) (end 101.2 112) (width 0.25) (layer "B.Cu") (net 9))
 (segment (start 101.2 112) (end 104.4 115.2) (width 0.25) (layer "B.Cu") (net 9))
 (segment (start 107.35 115.875) (end 108.1 115.875) (width 0.25) (layer "F.Cu") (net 12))
 (segment (start 108.1 115.875) (end 108.225 116) (width 0.25) (layer "F.Cu") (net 12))
 (segment (start 111.865 120.455) (end 112.51 121.1) (width 0.25) (layer "F.Cu") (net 12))
 (segment (start 112.335 108.665) (end 113.7 107.3) (width 0.25) (layer "F.Cu") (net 12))
 (segment (start 113.7 107.3) (end 114.8 107.3) (width 0.25) (layer "F.Cu") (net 12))
 (segment (start 115.153604 114.4) (end 109.525 114.4) (width 0.25) (layer "F.Cu") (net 12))
 (segment (start 111.875 108.665) (end 112.335 108.665) (width 0.25) (layer "F.Cu") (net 12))
 (segment (start 112.51 122.09) (end 113.5 123.08) (width 0.25) (layer "F.Cu") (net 12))
 (segment (start 108.225 117.625) (end 111.055 120.455) (width 0.25) (layer "F.Cu") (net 12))
 (segment (start 108.05 115.875) (end 107.35 115.875) (width 0.25) (layer "F.Cu") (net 12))
 (segment (start 114.8 107.3) (end 116.1 108.6) (width 0.25) (layer "F.Cu") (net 12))
 (segment (start 116.1 113.453604) (end 115.153604 114.4) (width 0.25) (layer "F.Cu") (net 12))
 (segment (start 116.1 108.6) (end 116.1 113.453604) (width 0.25) (layer "F.Cu") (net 12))
 (segment (start 112.51 121.1) (end 112.51 122.09) (width 0.25) (layer "F.Cu") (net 12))
 (segment (start 109.525 114.4) (end 108.05 115.875) (width 0.25) (layer "F.Cu") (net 12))
 (segment (start 111.055 120.455) (end 111.865 120.455) (width 0.25) (layer "F.Cu") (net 12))
 (segment (start 111.875 108.665) (end 112.635 108.665) (width 0.25) (layer "F.Cu") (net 12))
 (segment (start 108.225 116) (end 108.225 117.625) (width 0.25) (layer "F.Cu") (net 12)))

